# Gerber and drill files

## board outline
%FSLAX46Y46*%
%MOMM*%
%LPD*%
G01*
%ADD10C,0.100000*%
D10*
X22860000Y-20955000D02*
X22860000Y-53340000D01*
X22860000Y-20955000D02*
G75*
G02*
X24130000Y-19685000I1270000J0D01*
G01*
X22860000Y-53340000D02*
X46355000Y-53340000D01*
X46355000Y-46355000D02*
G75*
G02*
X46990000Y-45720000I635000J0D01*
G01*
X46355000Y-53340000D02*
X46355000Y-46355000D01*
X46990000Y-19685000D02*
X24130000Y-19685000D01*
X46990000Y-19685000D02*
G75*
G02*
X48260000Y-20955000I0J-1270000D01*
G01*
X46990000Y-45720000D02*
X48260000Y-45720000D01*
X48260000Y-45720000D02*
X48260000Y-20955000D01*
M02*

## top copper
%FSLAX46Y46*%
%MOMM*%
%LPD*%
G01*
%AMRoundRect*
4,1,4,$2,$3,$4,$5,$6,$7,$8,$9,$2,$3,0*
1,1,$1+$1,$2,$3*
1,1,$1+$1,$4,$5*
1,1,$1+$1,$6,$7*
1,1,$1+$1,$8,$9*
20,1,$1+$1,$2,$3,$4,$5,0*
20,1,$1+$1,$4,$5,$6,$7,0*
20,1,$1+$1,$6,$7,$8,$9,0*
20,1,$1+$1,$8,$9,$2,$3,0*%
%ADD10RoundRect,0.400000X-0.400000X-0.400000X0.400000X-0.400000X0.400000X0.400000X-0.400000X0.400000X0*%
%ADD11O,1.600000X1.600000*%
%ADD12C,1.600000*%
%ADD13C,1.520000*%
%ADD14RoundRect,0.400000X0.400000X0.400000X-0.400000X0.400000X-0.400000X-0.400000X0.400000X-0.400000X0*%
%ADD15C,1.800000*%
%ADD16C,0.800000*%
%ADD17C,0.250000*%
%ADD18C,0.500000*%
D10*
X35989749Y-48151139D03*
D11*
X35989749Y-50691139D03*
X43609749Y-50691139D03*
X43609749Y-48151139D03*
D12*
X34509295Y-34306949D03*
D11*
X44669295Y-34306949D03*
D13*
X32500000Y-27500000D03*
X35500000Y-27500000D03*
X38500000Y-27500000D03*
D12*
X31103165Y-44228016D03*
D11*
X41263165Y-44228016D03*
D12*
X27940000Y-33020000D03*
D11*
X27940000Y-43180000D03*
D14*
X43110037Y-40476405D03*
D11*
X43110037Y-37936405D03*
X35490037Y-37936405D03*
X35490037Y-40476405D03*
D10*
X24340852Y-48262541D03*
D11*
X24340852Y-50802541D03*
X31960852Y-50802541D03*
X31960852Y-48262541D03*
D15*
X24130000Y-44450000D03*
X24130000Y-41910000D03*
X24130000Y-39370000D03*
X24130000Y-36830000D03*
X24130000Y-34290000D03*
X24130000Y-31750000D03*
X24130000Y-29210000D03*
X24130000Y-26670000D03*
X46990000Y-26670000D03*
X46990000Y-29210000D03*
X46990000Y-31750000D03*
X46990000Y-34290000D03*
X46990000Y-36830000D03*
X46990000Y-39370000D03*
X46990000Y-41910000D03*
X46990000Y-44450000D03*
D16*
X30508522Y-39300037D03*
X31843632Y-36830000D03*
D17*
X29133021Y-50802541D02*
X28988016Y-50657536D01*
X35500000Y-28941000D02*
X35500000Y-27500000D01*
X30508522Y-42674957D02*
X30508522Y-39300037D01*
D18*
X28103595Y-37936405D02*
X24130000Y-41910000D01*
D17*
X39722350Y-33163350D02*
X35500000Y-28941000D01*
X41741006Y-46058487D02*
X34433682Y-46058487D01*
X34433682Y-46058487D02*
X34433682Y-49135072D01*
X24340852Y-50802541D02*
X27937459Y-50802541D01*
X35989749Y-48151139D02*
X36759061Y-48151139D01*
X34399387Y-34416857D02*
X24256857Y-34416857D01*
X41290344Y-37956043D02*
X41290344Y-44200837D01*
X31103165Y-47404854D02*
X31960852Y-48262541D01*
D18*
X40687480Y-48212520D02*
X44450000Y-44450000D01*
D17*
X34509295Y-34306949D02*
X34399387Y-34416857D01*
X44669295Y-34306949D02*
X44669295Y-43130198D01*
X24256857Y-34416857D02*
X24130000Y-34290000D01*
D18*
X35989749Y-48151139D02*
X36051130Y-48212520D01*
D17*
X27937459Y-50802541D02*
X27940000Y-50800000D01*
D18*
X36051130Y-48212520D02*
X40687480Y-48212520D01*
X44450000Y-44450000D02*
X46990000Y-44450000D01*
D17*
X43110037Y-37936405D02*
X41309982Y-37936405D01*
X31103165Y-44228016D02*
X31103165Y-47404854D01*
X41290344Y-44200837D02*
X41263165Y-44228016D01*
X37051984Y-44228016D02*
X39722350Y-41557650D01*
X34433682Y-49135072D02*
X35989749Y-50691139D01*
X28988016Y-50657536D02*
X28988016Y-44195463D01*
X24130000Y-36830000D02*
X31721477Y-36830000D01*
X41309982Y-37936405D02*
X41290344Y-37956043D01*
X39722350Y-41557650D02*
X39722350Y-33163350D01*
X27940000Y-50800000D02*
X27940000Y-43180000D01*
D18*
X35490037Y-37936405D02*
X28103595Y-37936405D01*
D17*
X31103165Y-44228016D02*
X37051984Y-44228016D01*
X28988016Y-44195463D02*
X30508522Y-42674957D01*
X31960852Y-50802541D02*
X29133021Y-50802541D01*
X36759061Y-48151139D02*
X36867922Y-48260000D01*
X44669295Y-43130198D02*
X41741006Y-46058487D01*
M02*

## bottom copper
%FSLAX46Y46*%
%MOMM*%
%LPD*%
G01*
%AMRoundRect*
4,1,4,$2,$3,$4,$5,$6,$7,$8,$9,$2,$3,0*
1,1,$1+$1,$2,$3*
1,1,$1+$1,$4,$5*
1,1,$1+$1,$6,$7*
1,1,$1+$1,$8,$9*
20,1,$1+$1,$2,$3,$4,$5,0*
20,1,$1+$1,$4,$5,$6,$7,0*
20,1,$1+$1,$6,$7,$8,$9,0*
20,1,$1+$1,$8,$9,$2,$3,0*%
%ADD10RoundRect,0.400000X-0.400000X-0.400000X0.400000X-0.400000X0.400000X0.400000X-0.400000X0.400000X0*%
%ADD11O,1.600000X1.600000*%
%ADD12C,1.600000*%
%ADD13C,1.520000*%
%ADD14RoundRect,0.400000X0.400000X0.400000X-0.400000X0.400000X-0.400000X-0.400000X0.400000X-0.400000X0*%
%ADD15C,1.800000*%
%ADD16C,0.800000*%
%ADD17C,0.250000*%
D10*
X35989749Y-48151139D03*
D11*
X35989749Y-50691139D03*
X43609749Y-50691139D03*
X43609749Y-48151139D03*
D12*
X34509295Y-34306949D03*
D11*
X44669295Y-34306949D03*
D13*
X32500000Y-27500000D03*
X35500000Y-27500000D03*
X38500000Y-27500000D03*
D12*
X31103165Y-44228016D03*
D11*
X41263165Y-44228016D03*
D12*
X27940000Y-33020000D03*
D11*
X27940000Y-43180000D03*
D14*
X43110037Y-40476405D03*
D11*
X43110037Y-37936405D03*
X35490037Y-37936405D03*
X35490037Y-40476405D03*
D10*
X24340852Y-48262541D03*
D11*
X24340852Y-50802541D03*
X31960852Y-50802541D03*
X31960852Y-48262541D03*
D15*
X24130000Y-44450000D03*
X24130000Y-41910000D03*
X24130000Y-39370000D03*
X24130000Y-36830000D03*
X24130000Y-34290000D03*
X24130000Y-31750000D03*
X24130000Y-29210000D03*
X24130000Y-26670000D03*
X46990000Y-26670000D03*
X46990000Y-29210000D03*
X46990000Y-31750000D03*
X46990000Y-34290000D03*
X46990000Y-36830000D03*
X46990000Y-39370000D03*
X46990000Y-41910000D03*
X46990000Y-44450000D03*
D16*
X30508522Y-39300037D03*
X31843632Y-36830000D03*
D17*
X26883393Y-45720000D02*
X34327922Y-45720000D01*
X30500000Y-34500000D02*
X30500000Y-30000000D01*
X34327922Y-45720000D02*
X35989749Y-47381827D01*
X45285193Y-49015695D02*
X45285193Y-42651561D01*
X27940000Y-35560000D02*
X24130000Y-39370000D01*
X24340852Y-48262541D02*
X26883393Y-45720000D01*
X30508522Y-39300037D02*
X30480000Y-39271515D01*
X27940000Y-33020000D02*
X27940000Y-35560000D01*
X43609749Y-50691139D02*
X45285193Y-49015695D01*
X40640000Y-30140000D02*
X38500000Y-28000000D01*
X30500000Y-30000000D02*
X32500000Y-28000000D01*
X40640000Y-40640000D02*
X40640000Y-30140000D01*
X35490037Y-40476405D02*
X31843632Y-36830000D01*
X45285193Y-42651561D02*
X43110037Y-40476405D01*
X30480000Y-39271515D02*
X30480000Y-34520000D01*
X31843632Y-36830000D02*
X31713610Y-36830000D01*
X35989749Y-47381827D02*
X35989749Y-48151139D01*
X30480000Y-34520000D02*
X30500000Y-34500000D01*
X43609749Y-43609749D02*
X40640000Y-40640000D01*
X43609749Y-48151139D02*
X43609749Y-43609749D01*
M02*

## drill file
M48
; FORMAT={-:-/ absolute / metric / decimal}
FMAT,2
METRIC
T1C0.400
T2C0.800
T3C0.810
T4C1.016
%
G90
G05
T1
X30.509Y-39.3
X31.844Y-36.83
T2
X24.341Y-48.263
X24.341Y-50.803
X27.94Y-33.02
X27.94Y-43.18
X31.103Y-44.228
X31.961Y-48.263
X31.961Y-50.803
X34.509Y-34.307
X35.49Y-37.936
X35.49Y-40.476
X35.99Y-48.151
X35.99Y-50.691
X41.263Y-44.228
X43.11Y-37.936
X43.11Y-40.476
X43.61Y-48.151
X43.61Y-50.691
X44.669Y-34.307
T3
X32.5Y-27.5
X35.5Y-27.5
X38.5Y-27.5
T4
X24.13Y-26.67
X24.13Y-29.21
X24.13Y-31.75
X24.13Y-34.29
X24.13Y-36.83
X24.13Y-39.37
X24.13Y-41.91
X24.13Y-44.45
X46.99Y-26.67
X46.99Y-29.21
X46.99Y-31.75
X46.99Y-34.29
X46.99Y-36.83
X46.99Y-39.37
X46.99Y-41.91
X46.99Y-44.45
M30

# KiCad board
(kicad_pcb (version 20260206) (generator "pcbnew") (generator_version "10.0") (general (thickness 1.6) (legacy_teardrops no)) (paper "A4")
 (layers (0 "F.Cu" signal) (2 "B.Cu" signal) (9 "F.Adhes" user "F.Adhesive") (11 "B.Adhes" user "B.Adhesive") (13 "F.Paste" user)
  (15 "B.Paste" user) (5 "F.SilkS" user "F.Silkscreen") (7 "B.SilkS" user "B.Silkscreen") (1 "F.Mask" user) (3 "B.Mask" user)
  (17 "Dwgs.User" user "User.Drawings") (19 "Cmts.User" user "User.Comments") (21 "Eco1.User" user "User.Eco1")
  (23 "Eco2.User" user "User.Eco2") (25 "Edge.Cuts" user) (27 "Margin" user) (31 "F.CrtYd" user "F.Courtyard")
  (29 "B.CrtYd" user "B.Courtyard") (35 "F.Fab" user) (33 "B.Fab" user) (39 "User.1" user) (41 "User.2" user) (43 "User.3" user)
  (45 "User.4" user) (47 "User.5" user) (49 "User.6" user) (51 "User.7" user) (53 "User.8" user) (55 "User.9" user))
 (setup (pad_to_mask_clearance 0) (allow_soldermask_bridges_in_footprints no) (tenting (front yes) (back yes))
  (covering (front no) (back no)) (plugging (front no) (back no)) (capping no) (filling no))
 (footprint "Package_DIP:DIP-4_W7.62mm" (layer "F.Cu") (at 35.989749 48.151139)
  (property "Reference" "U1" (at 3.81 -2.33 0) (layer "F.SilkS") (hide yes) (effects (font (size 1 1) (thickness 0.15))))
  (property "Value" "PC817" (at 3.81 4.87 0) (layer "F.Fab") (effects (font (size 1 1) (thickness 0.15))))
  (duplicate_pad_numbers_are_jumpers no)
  (pad "1" thru_hole roundrect (at 0 0) (size 1.6 1.6) (drill 0.8) (layers "*.Cu" "*.Mask") (remove_unused_layers no)
   (roundrect_rratio 0.25))
  (pad "2" thru_hole oval (at 0 2.54) (size 1.6 1.6) (drill 0.8) (layers "*.Cu" "*.Mask") (remove_unused_layers no))
  (pad "3" thru_hole oval (at 7.62 2.54) (size 1.6 1.6) (drill 0.8) (layers "*.Cu" "*.Mask") (remove_unused_layers no))
  (pad "4" thru_hole oval (at 7.62 0) (size 1.6 1.6) (drill 0.8) (layers "*.Cu" "*.Mask") (remove_unused_layers no)))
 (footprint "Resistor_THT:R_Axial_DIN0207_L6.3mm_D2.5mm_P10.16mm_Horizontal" (layer "F.Cu") (at 34.509295 34.306949)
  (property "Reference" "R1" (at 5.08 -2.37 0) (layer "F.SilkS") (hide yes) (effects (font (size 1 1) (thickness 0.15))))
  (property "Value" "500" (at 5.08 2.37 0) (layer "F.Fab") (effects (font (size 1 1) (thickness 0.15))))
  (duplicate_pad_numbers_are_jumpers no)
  (pad "1" thru_hole circle (at 0 0) (size 1.6 1.6) (drill 0.8) (layers "*.Cu" "*.Mask") (remove_unused_layers no))
  (pad "2" thru_hole oval (at 10.16 0) (size 1.6 1.6) (drill 0.8) (layers "*.Cu" "*.Mask") (remove_unused_layers no)))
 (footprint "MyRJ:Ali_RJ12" (layer "F.Cu") (at 34.5 25.5 180)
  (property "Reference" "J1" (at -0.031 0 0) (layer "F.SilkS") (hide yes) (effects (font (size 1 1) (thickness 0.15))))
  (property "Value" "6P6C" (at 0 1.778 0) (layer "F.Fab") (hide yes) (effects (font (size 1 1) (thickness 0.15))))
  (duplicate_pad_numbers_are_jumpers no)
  (pad "1" thru_hole circle (at 2 -2) (size 1.52 1.52) (drill 0.81) (layers "*.Cu" "*.Mask") (remove_unused_layers no))
  (pad "2" thru_hole circle (at -1 -2) (size 1.52 1.52) (drill 0.81) (layers "*.Cu" "*.Mask") (remove_unused_layers no))
  (pad "3" thru_hole circle (at -4 -2) (size 1.52 1.52) (drill 0.81) (layers "*.Cu" "*.Mask") (remove_unused_layers no)))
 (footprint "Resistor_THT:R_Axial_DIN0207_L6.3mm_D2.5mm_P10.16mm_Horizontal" (layer "F.Cu") (at 31.103165 44.228016)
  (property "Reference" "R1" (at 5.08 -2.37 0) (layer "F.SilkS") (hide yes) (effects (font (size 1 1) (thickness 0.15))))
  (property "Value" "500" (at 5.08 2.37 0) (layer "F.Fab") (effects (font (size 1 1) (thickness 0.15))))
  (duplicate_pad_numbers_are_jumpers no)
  (pad "1" thru_hole circle (at 0 0) (size 1.6 1.6) (drill 0.8) (layers "*.Cu" "*.Mask") (remove_unused_layers no))
  (pad "2" thru_hole oval (at 10.16 0) (size 1.6 1.6) (drill 0.8) (layers "*.Cu" "*.Mask") (remove_unused_layers no)))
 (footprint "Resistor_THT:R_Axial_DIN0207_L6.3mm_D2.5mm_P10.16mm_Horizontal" (layer "F.Cu") (at 27.94 33.02 -90)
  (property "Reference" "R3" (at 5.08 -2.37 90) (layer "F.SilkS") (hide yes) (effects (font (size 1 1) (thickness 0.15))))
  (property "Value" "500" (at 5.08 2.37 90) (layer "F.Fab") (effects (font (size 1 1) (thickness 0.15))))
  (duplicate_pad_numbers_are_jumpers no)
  (pad "1" thru_hole circle (at 0 0 270) (size 1.6 1.6) (drill 0.8) (layers "*.Cu" "*.Mask") (remove_unused_layers no))
  (pad "2" thru_hole oval (at 10.16 0 270) (size 1.6 1.6) (drill 0.8) (layers "*.Cu" "*.Mask") (remove_unused_layers no)))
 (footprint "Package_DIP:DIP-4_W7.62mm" (layer "F.Cu") (at 43.110037 40.476405 180)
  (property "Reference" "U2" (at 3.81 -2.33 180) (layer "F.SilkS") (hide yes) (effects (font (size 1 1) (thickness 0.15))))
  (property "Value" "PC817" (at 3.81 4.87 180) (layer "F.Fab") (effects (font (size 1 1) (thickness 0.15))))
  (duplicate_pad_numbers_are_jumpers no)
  (pad "1" thru_hole roundrect (at 0 0 180) (size 1.6 1.6) (drill 0.8) (layers "*.Cu" "*.Mask") (remove_unused_layers no)
   (roundrect_rratio 0.25))
  (pad "2" thru_hole oval (at 0 2.54 180) (size 1.6 1.6) (drill 0.8) (layers "*.Cu" "*.Mask") (remove_unused_layers no))
  (pad "3" thru_hole oval (at 7.62 2.54 180) (size 1.6 1.6) (drill 0.8) (layers "*.Cu" "*.Mask") (remove_unused_layers no))
  (pad "4" thru_hole oval (at 7.62 0 180) (size 1.6 1.6) (drill 0.8) (layers "*.Cu" "*.Mask") (remove_unused_layers no)))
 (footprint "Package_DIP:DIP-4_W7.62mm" (layer "F.Cu") (at 24.340852 48.262541)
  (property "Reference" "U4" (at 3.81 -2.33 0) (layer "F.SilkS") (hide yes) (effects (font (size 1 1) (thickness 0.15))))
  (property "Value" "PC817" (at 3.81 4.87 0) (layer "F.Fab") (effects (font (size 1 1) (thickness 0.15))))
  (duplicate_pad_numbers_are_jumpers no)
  (pad "1" thru_hole roundrect (at 0 0) (size 1.6 1.6) (drill 0.8) (layers "*.Cu" "*.Mask") (remove_unused_layers no)
   (roundrect_rratio 0.25))
  (pad "2" thru_hole oval (at 0 2.54) (size 1.6 1.6) (drill 0.8) (layers "*.Cu" "*.Mask") (remove_unused_layers no))
  (pad "3" thru_hole oval (at 7.62 2.54) (size 1.6 1.6) (drill 0.8) (layers "*.Cu" "*.Mask") (remove_unused_layers no))
  (pad "4" thru_hole oval (at 7.62 0) (size 1.6 1.6) (drill 0.8) (layers "*.Cu" "*.Mask") (remove_unused_layers no)))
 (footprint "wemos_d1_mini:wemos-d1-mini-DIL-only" (layer "B.Cu") (at 35.56 35.56 90)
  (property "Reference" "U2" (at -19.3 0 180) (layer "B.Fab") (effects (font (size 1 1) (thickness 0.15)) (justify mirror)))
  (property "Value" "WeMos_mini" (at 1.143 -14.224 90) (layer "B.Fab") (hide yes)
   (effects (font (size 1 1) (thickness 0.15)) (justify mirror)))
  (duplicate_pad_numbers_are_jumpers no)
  (pad "1" thru_hole circle (at -8.89 -11.43 90) (size 1.8 1.8) (drill 1.016) (layers "*.Cu" "*.Mask") (remove_unused_layers no))
  (pad "2" thru_hole circle (at -6.35 -11.43 90) (size 1.8 1.8) (drill 1.016) (layers "*.Cu" "*.Mask") (remove_unused_layers no))
  (pad "3" thru_hole circle (at -3.81 -11.43 90) (size 1.8 1.8) (drill 1.016) (layers "*.Cu" "*.Mask") (remove_unused_layers no))
  (pad "4" thru_hole circle (at -1.27 -11.43 90) (size 1.8 1.8) (drill 1.016) (layers "*.Cu" "*.Mask") (remove_unused_layers no))
  (pad "5" thru_hole circle (at 1.27 -11.43 90) (size 1.8 1.8) (drill 1.016) (layers "*.Cu" "*.Mask") (remove_unused_layers no))
  (pad "6" thru_hole circle (at 3.81 -11.43 90) (size 1.8 1.8) (drill 1.016) (layers "*.Cu" "*.Mask") (remove_unused_layers no))
  (pad "7" thru_hole circle (at 6.35 -11.43 90) (size 1.8 1.8) (drill 1.016) (layers "*.Cu" "*.Mask") (remove_unused_layers no))
  (pad "8" thru_hole circle (at 8.89 -11.43 90) (size 1.8 1.8) (drill 1.016) (layers "*.Cu" "*.Mask") (remove_unused_layers no))
  (pad "9" thru_hole circle (at 8.89 11.43 90) (size 1.8 1.8) (drill 1.016) (layers "*.Cu" "*.Mask") (remove_unused_layers no))
  (pad "10" thru_hole circle (at 6.35 11.43 90) (size 1.8 1.8) (drill 1.016) (layers "*.Cu" "*.Mask") (remove_unused_layers no))
  (pad "11" thru_hole circle (at 3.81 11.43 90) (size 1.8 1.8) (drill 1.016) (layers "*.Cu" "*.Mask") (remove_unused_layers no))
  (pad "12" thru_hole circle (at 1.27 11.43 90) (size 1.8 1.8) (drill 1.016) (layers "*.Cu" "*.Mask") (remove_unused_layers no))
  (pad "13" thru_hole circle (at -1.27 11.43 90) (size 1.8 1.8) (drill 1.016) (layers "*.Cu" "*.Mask") (remove_unused_layers no))
  (pad "14" thru_hole circle (at -3.81 11.43 90) (size 1.8 1.8) (drill 1.016) (layers "*.Cu" "*.Mask") (remove_unused_layers no))
  (pad "15" thru_hole circle (at -6.35 11.43 90) (size 1.8 1.8) (drill 1.016) (layers "*.Cu" "*.Mask") (remove_unused_layers no))
  (pad "16" thru_hole circle (at -8.89 11.43 90) (size 1.8 1.8) (drill 1.016) (layers "*.Cu" "*.Mask") (remove_unused_layers no)))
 (gr_line (start 22.86 20.955) (end 22.86 53.34) (stroke (width 0.1) (type solid)) (layer "Edge.Cuts"))
 (gr_arc (start 22.86 20.955) (mid 23.231974 20.056974) (end 24.13 19.685) (stroke (width 0.1) (type solid)) (layer "Edge.Cuts"))
 (gr_line (start 22.86 53.34) (end 46.355 53.34) (stroke (width 0.1) (type solid)) (layer "Edge.Cuts"))
 (gr_arc (start 46.355 46.355) (mid 46.540987 45.905987) (end 46.99 45.72) (stroke (width 0.1) (type solid)) (layer "Edge.Cuts"))
 (gr_line (start 46.355 53.34) (end 46.355 46.355) (stroke (width 0.1) (type solid)) (layer "Edge.Cuts"))
 (gr_line (start 46.99 19.685) (end 24.13 19.685) (stroke (width 0.1) (type solid)) (layer "Edge.Cuts"))
 (gr_arc (start 46.99 19.685) (mid 47.888026 20.056974) (end 48.26 20.955) (stroke (width 0.1) (type solid)) (layer "Edge.Cuts"))
 (gr_line (start 46.99 45.72) (end 48.26 45.72) (stroke (width 0.1) (type solid)) (layer "Edge.Cuts"))
 (gr_line (start 48.26 45.72) (end 48.26 20.955) (stroke (width 0.1) (type solid)) (layer "Edge.Cuts"))
 (segment (start 29.133021 50.802541) (end 28.988016 50.657536) (width 0.25) (layer "F.Cu") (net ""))
 (segment (start 35.5 28.941) (end 35.5 27.5) (width 0.25) (layer "F.Cu") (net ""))
 (segment (start 30.508522 42.674957) (end 30.508522 39.300037) (width 0.25) (layer "F.Cu") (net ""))
 (segment (start 28.103595 37.936405) (end 24.13 41.91) (width 0.5) (layer "F.Cu") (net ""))
 (segment (start 39.72235 33.16335) (end 35.5 28.941) (width 0.25) (layer "F.Cu") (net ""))
 (segment (start 41.741006 46.058487) (end 34.433682 46.058487) (width 0.25) (layer "F.Cu") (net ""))
 (segment (start 34.433682 46.058487) (end 34.433682 49.135072) (width 0.25) (layer "F.Cu") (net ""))
 (segment (start 24.340852 50.802541) (end 27.937459 50.802541) (width 0.25) (layer "F.Cu") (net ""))
 (segment (start 35.989749 48.151139) (end 36.759061 48.151139) (width 0.25) (layer "F.Cu") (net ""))
 (segment (start 34.399387 34.416857) (end 24.256857 34.416857) (width 0.25) (layer "F.Cu") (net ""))
 (segment (start 41.290344 37.956043) (end 41.290344 44.200837) (width 0.25) (layer "F.Cu") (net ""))
 (segment (start 31.103165 47.404854) (end 31.960852 48.262541) (width 0.25) (layer "F.Cu") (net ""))
 (segment (start 40.68748 48.21252) (end 44.45 44.45) (width 0.5) (layer "F.Cu") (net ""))
 (segment (start 34.509295 34.306949) (end 34.399387 34.416857) (width 0.25) (layer "F.Cu") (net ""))
 (segment (start 44.669295 34.306949) (end 44.669295 43.130198) (width 0.25) (layer "F.Cu") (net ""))
 (segment (start 24.256857 34.416857) (end 24.13 34.29) (width 0.25) (layer "F.Cu") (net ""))
 (segment (start 35.989749 48.151139) (end 36.05113 48.21252) (width 0.5) (layer "F.Cu") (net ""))
 (segment (start 27.937459 50.802541) (end 27.94 50.8) (width 0.25) (layer "F.Cu") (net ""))
 (segment (start 36.05113 48.21252) (end 40.68748 48.21252) (width 0.5) (layer "F.Cu") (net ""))
 (segment (start 44.45 44.45) (end 46.99 44.45) (width 0.5) (layer "F.Cu") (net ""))
 (segment (start 43.110037 37.936405) (end 41.309982 37.936405) (width 0.25) (layer "F.Cu") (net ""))
 (segment (start 31.103165 44.228016) (end 31.103165 47.404854) (width 0.25) (layer "F.Cu") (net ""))
 (segment (start 41.290344 44.200837) (end 41.263165 44.228016) (width 0.25) (layer "F.Cu") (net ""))
 (segment (start 37.051984 44.228016) (end 39.72235 41.55765) (width 0.25) (layer "F.Cu") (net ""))
 (segment (start 34.433682 49.135072) (end 35.989749 50.691139) (width 0.25) (layer "F.Cu") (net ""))
 (segment (start 28.988016 50.657536) (end 28.988016 44.195463) (width 0.25) (layer "F.Cu") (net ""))
 (segment (start 24.13 36.83) (end 31.721477 36.83) (width 0.25) (layer "F.Cu") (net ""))
 (segment (start 41.309982 37.936405) (end 41.290344 37.956043) (width 0.25) (layer "F.Cu") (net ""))
 (segment (start 39.72235 41.55765) (end 39.72235 33.16335) (width 0.25) (layer "F.Cu") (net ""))
 (segment (start 27.94 50.8) (end 27.94 43.18) (width 0.25) (layer "F.Cu") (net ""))
 (segment (start 35.490037 37.936405) (end 28.103595 37.936405) (width 0.5) (layer "F.Cu") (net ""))
 (segment (start 31.103165 44.228016) (end 37.051984 44.228016) (width 0.25) (layer "F.Cu") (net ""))
 (segment (start 28.988016 44.195463) (end 30.508522 42.674957) (width 0.25) (layer "F.Cu") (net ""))
 (segment (start 31.960852 50.802541) (end 29.133021 50.802541) (width 0.25) (layer "F.Cu") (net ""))
 (segment (start 36.759061 48.151139) (end 36.867922 48.26) (width 0.25) (layer "F.Cu") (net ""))
 (segment (start 44.669295 43.130198) (end 41.741006 46.058487) (width 0.25) (layer "F.Cu") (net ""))
 (via (at 30.508522 39.300037) (size 0.8) (drill 0.4) (layers "F.Cu" "B.Cu") (capping no) (covering (front no) (back no))
  (plugging (front no) (back no)) (filling no) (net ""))
 (via (at 31.843632 36.83) (size 0.8) (drill 0.4) (layers "F.Cu" "B.Cu") (capping no) (covering (front no) (back no))
  (plugging (front no) (back no)) (filling no) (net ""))
 (segment (start 26.883393 45.72) (end 34.327922 45.72) (width 0.25) (layer "B.Cu") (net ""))
 (segment (start 30.5 34.5) (end 30.5 30) (width 0.25) (layer "B.Cu") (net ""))
 (segment (start 34.327922 45.72) (end 35.989749 47.381827) (width 0.25) (layer "B.Cu") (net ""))
 (segment (start 45.285193 49.015695) (end 45.285193 42.651561) (width 0.25) (layer "B.Cu") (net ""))
 (segment (start 27.94 35.56) (end 24.13 39.37) (width 0.25) (layer "B.Cu") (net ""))
 (segment (start 24.340852 48.262541) (end 26.883393 45.72) (width 0.25) (layer "B.Cu") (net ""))
 (segment (start 30.508522 39.300037) (end 30.48 39.271515) (width 0.25) (layer "B.Cu") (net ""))
 (segment (start 27.94 33.02) (end 27.94 35.56) (width 0.25) (layer "B.Cu") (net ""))
 (segment (start 43.609749 50.691139) (end 45.285193 49.015695) (width 0.25) (layer "B.Cu") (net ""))
 (segment (start 40.64 30.14) (end 38.5 28) (width 0.25) (layer "B.Cu") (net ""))
 (segment (start 30.5 30) (end 32.5 28) (width 0.25) (layer "B.Cu") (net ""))
 (segment (start 40.64 40.64) (end 40.64 30.14) (width 0.25) (layer "B.Cu") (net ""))
 (segment (start 35.490037 40.476405) (end 31.843632 36.83) (width 0.25) (layer "B.Cu") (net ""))
 (segment (start 45.285193 42.651561) (end 43.110037 40.476405) (width 0.25) (layer "B.Cu") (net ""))
 (segment (start 30.48 39.271515) (end 30.48 34.52) (width 0.25) (layer "B.Cu") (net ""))
 (segment (start 31.843632 36.83) (end 31.71361 36.83) (width 0.25) (layer "B.Cu") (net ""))
 (segment (start 35.989749 47.381827) (end 35.989749 48.151139) (width 0.25) (layer "B.Cu") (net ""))
 (segment (start 30.48 34.52) (end 30.5 34.5) (width 0.25) (layer "B.Cu") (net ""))
 (segment (start 43.609749 43.609749) (end 40.64 40.64) (width 0.25) (layer "B.Cu") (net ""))
 (segment (start 43.609749 48.151139) (end 43.609749 43.609749) (width 0.25) (layer "B.Cu") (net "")))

